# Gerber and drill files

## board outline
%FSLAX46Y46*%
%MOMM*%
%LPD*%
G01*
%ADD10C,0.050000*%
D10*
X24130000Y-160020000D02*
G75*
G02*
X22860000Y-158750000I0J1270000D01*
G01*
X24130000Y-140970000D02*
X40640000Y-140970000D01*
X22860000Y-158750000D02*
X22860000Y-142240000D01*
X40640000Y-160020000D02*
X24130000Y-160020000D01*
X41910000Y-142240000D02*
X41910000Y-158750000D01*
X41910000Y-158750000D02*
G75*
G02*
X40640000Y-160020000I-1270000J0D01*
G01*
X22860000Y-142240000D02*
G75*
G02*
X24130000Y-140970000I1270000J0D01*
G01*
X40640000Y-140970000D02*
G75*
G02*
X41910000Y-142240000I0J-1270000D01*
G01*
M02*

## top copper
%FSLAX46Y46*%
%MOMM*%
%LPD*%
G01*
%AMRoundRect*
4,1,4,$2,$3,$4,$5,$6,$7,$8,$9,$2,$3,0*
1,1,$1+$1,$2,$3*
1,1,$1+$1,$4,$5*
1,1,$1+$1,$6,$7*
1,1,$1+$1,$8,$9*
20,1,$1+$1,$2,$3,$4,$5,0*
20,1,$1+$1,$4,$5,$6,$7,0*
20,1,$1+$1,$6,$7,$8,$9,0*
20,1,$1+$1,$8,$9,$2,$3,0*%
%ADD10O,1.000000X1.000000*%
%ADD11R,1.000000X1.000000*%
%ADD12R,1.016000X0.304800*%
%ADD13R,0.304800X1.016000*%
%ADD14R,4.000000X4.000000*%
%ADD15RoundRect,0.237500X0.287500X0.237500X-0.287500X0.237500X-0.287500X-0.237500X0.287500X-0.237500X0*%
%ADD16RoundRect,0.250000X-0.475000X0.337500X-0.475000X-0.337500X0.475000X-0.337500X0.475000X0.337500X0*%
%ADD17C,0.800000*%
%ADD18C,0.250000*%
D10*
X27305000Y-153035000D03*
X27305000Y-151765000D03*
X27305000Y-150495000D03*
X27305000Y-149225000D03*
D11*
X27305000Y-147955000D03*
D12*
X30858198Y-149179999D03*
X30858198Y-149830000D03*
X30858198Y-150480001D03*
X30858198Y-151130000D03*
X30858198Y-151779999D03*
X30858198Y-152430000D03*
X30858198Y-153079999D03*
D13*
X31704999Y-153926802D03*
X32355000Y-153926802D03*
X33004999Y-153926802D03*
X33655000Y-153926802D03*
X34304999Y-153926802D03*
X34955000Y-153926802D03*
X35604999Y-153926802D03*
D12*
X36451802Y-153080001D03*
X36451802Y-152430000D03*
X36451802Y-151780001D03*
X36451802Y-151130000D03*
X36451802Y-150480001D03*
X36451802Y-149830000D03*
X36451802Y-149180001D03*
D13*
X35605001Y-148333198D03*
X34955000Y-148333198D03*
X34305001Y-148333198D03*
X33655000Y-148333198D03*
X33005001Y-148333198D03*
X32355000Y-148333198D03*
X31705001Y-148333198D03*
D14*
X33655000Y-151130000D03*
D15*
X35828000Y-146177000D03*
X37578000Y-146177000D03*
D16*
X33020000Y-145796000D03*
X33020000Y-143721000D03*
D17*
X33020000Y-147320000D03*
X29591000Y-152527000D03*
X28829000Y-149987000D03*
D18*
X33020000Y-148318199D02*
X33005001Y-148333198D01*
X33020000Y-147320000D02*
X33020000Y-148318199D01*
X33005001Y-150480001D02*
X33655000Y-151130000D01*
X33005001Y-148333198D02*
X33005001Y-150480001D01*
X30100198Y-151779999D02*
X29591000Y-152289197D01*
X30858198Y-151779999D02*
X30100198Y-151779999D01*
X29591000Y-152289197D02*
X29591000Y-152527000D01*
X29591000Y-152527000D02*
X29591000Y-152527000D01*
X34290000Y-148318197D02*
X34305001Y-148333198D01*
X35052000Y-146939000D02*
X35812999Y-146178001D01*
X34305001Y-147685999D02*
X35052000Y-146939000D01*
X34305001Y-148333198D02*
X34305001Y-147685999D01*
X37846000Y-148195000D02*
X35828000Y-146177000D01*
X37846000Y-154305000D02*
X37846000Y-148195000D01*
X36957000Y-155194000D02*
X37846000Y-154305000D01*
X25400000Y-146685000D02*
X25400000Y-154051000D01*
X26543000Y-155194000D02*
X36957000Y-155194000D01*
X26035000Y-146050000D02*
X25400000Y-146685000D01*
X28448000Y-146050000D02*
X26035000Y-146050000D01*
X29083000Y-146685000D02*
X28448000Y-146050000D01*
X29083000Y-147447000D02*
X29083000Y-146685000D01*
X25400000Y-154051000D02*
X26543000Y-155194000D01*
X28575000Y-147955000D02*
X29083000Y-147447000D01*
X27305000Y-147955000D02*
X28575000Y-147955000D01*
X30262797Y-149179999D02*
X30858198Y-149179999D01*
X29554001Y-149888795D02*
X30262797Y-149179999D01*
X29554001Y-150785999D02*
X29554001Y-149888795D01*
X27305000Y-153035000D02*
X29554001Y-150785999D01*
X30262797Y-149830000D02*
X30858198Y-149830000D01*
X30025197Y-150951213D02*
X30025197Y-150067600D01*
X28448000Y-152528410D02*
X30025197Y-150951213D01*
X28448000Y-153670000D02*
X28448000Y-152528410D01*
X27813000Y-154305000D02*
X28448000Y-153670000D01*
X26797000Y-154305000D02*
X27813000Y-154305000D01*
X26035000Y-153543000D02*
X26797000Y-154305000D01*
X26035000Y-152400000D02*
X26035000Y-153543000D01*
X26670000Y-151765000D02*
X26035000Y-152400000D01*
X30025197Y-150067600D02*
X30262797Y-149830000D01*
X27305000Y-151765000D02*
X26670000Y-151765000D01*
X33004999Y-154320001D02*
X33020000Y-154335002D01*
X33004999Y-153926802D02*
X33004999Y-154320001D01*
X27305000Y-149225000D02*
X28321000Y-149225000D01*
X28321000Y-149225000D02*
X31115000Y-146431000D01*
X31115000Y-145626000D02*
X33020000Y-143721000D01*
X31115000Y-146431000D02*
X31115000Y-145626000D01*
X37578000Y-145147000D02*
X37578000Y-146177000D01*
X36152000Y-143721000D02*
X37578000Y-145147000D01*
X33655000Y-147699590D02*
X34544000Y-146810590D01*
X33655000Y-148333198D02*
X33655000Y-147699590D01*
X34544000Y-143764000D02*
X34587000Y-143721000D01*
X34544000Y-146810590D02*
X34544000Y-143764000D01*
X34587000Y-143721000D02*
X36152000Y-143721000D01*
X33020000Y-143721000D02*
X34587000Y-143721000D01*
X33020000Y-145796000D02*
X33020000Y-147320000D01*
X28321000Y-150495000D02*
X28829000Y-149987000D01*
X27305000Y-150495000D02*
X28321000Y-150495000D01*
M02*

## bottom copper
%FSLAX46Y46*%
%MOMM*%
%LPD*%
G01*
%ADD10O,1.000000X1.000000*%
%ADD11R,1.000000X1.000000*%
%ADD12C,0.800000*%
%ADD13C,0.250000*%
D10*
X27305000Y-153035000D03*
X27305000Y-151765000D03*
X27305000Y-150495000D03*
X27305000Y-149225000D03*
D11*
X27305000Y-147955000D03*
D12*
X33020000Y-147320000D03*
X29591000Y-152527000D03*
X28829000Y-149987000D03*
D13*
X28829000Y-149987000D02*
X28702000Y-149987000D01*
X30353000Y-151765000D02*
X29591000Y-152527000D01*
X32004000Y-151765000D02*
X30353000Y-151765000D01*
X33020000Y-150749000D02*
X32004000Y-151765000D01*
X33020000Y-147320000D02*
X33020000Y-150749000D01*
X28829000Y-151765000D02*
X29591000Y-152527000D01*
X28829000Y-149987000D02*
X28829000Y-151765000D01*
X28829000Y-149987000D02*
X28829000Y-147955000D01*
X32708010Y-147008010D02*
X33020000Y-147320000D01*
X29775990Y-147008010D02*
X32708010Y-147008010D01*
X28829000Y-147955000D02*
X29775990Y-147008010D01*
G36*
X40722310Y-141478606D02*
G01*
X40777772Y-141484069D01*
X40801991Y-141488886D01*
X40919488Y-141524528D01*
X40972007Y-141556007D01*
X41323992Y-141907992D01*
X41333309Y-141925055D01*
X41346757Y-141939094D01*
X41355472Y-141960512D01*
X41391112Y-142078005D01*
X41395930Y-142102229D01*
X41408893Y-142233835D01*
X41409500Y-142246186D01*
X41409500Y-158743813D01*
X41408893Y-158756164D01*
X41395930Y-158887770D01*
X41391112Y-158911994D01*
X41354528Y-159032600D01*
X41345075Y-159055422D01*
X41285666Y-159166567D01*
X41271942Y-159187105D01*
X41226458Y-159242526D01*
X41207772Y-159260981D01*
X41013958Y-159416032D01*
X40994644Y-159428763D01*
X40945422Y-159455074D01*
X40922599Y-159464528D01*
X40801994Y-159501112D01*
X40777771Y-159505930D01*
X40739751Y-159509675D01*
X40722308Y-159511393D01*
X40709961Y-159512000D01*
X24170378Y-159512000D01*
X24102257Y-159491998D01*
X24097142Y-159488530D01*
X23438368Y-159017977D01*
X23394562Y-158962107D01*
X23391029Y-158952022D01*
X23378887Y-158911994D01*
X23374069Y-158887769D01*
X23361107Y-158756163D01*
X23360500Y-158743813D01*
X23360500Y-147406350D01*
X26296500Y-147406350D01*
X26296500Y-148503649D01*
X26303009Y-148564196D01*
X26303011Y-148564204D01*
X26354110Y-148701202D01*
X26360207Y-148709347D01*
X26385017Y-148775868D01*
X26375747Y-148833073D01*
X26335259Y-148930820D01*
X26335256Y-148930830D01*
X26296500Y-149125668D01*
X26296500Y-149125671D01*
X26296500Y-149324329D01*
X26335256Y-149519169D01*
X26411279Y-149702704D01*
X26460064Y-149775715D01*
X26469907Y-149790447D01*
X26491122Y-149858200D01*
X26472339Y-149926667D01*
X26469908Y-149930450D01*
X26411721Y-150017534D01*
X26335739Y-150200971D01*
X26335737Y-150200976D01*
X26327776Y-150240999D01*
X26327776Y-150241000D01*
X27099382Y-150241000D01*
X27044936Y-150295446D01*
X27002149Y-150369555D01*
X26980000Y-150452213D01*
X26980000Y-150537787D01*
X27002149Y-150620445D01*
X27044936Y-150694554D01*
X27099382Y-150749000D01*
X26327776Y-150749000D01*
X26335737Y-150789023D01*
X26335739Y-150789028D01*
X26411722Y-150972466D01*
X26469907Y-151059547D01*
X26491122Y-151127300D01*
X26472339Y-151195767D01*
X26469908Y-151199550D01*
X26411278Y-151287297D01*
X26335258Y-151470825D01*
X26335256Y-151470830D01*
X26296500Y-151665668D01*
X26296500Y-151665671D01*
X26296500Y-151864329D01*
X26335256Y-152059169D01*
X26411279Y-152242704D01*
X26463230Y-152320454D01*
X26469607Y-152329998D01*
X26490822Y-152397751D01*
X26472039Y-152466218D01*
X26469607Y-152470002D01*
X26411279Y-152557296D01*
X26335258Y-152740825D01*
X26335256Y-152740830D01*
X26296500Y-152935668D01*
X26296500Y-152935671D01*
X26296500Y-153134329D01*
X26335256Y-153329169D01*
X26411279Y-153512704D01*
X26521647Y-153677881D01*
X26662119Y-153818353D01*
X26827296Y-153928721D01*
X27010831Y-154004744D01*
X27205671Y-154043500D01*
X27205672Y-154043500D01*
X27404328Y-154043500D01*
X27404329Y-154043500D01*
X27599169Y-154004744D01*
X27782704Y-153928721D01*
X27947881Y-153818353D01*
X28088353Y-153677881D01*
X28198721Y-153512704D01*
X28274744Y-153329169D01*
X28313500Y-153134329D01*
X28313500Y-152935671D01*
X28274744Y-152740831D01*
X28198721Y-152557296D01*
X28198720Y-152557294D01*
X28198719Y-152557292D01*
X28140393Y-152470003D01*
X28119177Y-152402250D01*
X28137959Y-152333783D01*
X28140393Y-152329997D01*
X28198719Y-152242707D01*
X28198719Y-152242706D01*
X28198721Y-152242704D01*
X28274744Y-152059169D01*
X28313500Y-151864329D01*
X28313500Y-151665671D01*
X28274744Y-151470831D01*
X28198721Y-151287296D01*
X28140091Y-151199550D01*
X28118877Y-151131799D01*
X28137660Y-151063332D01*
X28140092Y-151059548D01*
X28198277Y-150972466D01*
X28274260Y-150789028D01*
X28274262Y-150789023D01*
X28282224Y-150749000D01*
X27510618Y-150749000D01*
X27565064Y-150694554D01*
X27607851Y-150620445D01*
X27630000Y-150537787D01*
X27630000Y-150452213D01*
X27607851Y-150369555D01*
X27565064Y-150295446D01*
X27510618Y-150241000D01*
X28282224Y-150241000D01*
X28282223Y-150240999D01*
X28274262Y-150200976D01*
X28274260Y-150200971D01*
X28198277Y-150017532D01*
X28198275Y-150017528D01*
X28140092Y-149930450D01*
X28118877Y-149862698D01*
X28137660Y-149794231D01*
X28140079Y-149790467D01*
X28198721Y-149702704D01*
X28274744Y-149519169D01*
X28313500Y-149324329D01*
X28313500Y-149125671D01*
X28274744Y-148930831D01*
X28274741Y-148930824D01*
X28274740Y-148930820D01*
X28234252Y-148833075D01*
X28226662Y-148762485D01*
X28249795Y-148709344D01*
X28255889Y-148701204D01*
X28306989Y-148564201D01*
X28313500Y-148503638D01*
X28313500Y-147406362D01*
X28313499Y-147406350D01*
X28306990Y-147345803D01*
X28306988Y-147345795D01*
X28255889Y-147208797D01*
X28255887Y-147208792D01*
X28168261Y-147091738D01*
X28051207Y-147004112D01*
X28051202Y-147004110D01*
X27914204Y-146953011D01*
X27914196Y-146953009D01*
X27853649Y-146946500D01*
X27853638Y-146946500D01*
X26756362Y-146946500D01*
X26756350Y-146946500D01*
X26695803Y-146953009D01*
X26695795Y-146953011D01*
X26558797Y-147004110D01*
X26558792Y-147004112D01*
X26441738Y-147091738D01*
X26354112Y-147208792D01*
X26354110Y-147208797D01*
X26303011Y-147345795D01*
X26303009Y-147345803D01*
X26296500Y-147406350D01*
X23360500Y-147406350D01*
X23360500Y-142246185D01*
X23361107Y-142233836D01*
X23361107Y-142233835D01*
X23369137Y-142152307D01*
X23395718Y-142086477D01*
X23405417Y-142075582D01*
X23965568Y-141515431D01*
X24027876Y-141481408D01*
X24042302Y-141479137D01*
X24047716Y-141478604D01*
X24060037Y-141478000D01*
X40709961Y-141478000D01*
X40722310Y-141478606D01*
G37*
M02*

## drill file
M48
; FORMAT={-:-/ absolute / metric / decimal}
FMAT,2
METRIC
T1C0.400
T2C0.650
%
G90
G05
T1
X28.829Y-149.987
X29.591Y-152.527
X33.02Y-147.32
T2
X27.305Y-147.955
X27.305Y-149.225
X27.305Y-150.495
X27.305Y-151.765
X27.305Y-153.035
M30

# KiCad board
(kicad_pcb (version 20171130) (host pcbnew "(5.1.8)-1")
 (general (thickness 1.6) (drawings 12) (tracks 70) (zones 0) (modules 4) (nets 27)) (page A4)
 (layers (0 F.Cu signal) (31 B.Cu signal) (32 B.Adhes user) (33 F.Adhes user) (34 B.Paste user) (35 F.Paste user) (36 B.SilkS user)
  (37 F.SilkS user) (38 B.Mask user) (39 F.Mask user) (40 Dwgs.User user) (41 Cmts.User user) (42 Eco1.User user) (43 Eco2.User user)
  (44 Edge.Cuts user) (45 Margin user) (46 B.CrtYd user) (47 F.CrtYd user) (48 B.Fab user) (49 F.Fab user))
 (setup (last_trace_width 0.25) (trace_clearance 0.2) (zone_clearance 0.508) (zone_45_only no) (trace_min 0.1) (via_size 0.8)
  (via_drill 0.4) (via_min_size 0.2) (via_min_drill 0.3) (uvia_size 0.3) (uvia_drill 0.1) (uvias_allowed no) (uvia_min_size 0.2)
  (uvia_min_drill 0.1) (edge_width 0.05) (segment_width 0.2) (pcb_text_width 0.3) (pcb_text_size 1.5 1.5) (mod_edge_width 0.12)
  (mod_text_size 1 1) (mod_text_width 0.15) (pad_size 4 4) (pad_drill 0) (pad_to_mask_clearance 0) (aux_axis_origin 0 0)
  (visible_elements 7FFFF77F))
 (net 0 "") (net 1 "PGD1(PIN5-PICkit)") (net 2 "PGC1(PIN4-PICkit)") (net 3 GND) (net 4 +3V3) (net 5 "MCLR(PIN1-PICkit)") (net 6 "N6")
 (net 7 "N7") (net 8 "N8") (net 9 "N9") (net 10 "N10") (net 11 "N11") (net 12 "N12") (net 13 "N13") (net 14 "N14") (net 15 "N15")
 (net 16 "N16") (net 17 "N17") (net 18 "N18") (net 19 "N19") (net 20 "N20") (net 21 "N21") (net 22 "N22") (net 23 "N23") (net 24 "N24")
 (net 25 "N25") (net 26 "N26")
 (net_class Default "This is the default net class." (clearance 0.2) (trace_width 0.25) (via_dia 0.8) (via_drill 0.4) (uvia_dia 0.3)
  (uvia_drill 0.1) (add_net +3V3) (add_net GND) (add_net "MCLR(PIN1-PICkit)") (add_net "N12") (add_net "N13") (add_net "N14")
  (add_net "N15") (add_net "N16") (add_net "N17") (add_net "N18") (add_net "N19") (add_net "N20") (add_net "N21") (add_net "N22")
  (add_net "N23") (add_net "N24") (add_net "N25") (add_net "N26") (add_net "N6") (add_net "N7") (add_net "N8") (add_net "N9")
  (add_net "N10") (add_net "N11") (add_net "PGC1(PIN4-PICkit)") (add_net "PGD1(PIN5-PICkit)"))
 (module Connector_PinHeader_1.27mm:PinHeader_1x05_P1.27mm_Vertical (layer F.Cu) (at 27.305 147.955)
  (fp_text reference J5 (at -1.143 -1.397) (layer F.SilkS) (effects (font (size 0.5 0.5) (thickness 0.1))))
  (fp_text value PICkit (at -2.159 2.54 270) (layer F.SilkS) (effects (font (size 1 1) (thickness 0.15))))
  (pad 5 thru_hole oval (at 0 5.08) (size 1 1) (drill 0.65) (layers *.Cu *.Mask) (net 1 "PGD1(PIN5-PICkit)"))
  (pad 4 thru_hole oval (at 0 3.81) (size 1 1) (drill 0.65) (layers *.Cu *.Mask) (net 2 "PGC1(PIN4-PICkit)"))
  (pad 3 thru_hole oval (at 0 2.54) (size 1 1) (drill 0.65) (layers *.Cu *.Mask) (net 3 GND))
  (pad 2 thru_hole oval (at 0 1.27) (size 1 1) (drill 0.65) (layers *.Cu *.Mask) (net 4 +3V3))
  (pad 1 thru_hole rect (at 0 0) (size 1 1) (drill 0.65) (layers *.Cu *.Mask) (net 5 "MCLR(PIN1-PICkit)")))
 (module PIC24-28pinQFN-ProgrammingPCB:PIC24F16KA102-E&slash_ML (layer F.Cu) (at 33.655 151.13)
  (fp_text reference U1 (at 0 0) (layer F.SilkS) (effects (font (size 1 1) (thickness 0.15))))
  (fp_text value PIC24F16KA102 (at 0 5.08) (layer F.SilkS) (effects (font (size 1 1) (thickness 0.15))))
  (pad 1 smd rect (at -2.796802 -1.950001 90) (size 0.3048 1.016) (layers F.Cu F.Paste F.Mask) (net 1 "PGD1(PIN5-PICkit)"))
  (pad 2 smd rect (at -2.796802 -1.3 90) (size 0.3048 1.016) (layers F.Cu F.Paste F.Mask) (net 2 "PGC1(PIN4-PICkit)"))
  (pad 3 smd rect (at -2.796802 -0.649999 90) (size 0.3048 1.016) (layers F.Cu F.Paste F.Mask) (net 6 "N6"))
  (pad 4 smd rect (at -2.796802 0 90) (size 0.3048 1.016) (layers F.Cu F.Paste F.Mask) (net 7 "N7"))
  (pad 5 smd rect (at -2.796802 0.649999 90) (size 0.3048 1.016) (layers F.Cu F.Paste F.Mask) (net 3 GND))
  (pad 6 smd rect (at -2.796802 1.3 90) (size 0.3048 1.016) (layers F.Cu F.Paste F.Mask) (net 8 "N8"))
  (pad 7 smd rect (at -2.796802 1.949999 90) (size 0.3048 1.016) (layers F.Cu F.Paste F.Mask) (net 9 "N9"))
  (pad 8 smd rect (at -1.950001 2.796802) (size 0.3048 1.016) (layers F.Cu F.Paste F.Mask) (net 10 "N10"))
  (pad 9 smd rect (at -1.3 2.796802) (size 0.3048 1.016) (layers F.Cu F.Paste F.Mask) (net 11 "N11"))
  (pad 10 smd rect (at -0.650001 2.796802) (size 0.3048 1.016) (layers F.Cu F.Paste F.Mask) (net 4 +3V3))
  (pad 11 smd rect (at 0 2.796802) (size 0.3048 1.016) (layers F.Cu F.Paste F.Mask) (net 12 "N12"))
  (pad 12 smd rect (at 0.649999 2.796802) (size 0.3048 1.016) (layers F.Cu F.Paste F.Mask) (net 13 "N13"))
  (pad 13 smd rect (at 1.3 2.796802) (size 0.3048 1.016) (layers F.Cu F.Paste F.Mask) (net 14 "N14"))
  (pad 14 smd rect (at 1.949999 2.796802) (size 0.3048 1.016) (layers F.Cu F.Paste F.Mask) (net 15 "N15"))
  (pad 15 smd rect (at 2.796802 1.950001 90) (size 0.3048 1.016) (layers F.Cu F.Paste F.Mask) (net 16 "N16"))
  (pad 16 smd rect (at 2.796802 1.3 90) (size 0.3048 1.016) (layers F.Cu F.Paste F.Mask) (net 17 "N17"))
  (pad 17 smd rect (at 2.796802 0.650001 90) (size 0.3048 1.016) (layers F.Cu F.Paste F.Mask) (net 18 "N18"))
  (pad 18 smd rect (at 2.796802 0 90) (size 0.3048 1.016) (layers F.Cu F.Paste F.Mask) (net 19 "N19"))
  (pad 19 smd rect (at 2.796802 -0.649999 90) (size 0.3048 1.016) (layers F.Cu F.Paste F.Mask) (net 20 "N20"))
  (pad 20 smd rect (at 2.796802 -1.3 90) (size 0.3048 1.016) (layers F.Cu F.Paste F.Mask) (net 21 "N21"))
  (pad 21 smd rect (at 2.796802 -1.949999 90) (size 0.3048 1.016) (layers F.Cu F.Paste F.Mask) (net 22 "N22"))
  (pad 22 smd rect (at 1.950001 -2.796802) (size 0.3048 1.016) (layers F.Cu F.Paste F.Mask) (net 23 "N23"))
  (pad 23 smd rect (at 1.3 -2.796802) (size 0.3048 1.016) (layers F.Cu F.Paste F.Mask) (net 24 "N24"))
  (pad 24 smd rect (at 0.650001 -2.796802) (size 0.3048 1.016) (layers F.Cu F.Paste F.Mask) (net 5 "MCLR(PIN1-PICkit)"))
  (pad 25 smd rect (at 0 -2.796802) (size 0.3048 1.016) (layers F.Cu F.Paste F.Mask) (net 4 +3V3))
  (pad 26 smd rect (at -0.649999 -2.796802) (size 0.3048 1.016) (layers F.Cu F.Paste F.Mask) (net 3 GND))
  (pad 27 smd rect (at -1.3 -2.796802) (size 0.3048 1.016) (layers F.Cu F.Paste F.Mask) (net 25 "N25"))
  (pad 28 smd rect (at -1.949999 -2.796802) (size 0.3048 1.016) (layers F.Cu F.Paste F.Mask) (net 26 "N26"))
  (pad EP smd rect (at 0 0) (size 4 4) (layers F.Cu F.Paste F.Mask) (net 3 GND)))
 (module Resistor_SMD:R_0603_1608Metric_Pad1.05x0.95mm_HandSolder (layer F.Cu) (at 36.703 146.177 180)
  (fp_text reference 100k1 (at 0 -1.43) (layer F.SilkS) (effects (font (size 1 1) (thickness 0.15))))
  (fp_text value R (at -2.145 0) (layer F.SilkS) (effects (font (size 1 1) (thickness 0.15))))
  (pad 2 smd roundrect (at 0.875 0 180) (size 1.05 0.95) (layers F.Cu F.Paste F.Mask) (roundrect_rratio 0.25) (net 5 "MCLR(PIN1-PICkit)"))
  (pad 1 smd roundrect (at -0.875 0 180) (size 1.05 0.95) (layers F.Cu F.Paste F.Mask) (roundrect_rratio 0.25) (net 4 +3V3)))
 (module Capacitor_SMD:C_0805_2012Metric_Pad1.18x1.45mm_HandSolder (layer F.Cu) (at 33.02 144.7585 270)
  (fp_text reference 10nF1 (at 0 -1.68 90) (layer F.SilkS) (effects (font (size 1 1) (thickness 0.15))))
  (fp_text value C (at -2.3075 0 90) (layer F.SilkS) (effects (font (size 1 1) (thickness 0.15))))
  (pad 2 smd roundrect (at 1.0375 0 270) (size 1.175 1.45) (layers F.Cu F.Paste F.Mask) (roundrect_rratio 0.212766) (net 3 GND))
  (pad 1 smd roundrect (at -1.0375 0 270) (size 1.175 1.45) (layers F.Cu F.Paste F.Mask) (roundrect_rratio 0.212766) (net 4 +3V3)))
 (gr_arc (start 24.13 158.75) (end 22.86 158.75) (angle -90) (layer Edge.Cuts) (width 0.05))
 (gr_line (start 24.13 140.97) (end 40.64 140.97) (layer Edge.Cuts) (width 0.05))
 (gr_line (start 22.86 158.75) (end 22.86 142.24) (layer Edge.Cuts) (width 0.05))
 (gr_line (start 40.64 160.02) (end 24.13 160.02) (layer Edge.Cuts) (width 0.05))
 (gr_line (start 41.91 142.24) (end 41.91 158.75) (layer Edge.Cuts) (width 0.05))
 (gr_arc (start 40.64 158.75) (end 40.64 160.02) (angle -90) (layer Edge.Cuts) (width 0.05))
 (gr_arc (start 24.13 142.24) (end 24.13 140.97) (angle -90) (layer Edge.Cuts) (width 0.05))
 (gr_arc (start 40.64 142.24) (end 41.91 142.24) (angle -90) (layer Edge.Cuts) (width 0.05))
 (via (at 33.02 147.32) (size 0.8) (drill 0.4) (layers F.Cu B.Cu) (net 3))
 (segment (start 33.02 148.318199) (end 33.005001 148.333198) (width 0.25) (layer F.Cu) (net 3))
 (segment (start 33.02 147.32) (end 33.02 148.318199) (width 0.25) (layer F.Cu) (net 3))
 (segment (start 33.005001 150.480001) (end 33.655 151.13) (width 0.25) (layer F.Cu) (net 3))
 (segment (start 33.005001 148.333198) (end 33.005001 150.480001) (width 0.25) (layer F.Cu) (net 3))
 (segment (start 30.100198 151.779999) (end 29.591 152.289197) (width 0.25) (layer F.Cu) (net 3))
 (segment (start 30.858198 151.779999) (end 30.100198 151.779999) (width 0.25) (layer F.Cu) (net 3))
 (segment (start 29.591 152.289197) (end 29.591 152.527) (width 0.25) (layer F.Cu) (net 3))
 (segment (start 29.591 152.527) (end 29.591 152.527) (width 0.25) (layer F.Cu) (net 3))
 (via (at 29.591 152.527) (size 0.8) (drill 0.4) (layers F.Cu B.Cu) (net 3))
 (segment (start 34.29 148.318197) (end 34.305001 148.333198) (width 0.25) (layer F.Cu) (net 5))
 (segment (start 35.052 146.939) (end 35.812999 146.178001) (width 0.25) (layer F.Cu) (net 5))
 (segment (start 34.305001 147.685999) (end 35.052 146.939) (width 0.25) (layer F.Cu) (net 5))
 (segment (start 34.305001 148.333198) (end 34.305001 147.685999) (width 0.25) (layer F.Cu) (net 5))
 (segment (start 37.846 148.195) (end 35.828 146.177) (width 0.25) (layer F.Cu) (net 5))
 (segment (start 37.846 154.305) (end 37.846 148.195) (width 0.25) (layer F.Cu) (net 5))
 (segment (start 36.957 155.194) (end 37.846 154.305) (width 0.25) (layer F.Cu) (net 5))
 (segment (start 25.4 146.685) (end 25.4 154.051) (width 0.25) (layer F.Cu) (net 5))
 (segment (start 26.543 155.194) (end 36.957 155.194) (width 0.25) (layer F.Cu) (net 5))
 (segment (start 26.035 146.05) (end 25.4 146.685) (width 0.25) (layer F.Cu) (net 5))
 (segment (start 28.448 146.05) (end 26.035 146.05) (width 0.25) (layer F.Cu) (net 5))
 (segment (start 29.083 146.685) (end 28.448 146.05) (width 0.25) (layer F.Cu) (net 5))
 (segment (start 29.083 147.447) (end 29.083 146.685) (width 0.25) (layer F.Cu) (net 5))
 (segment (start 25.4 154.051) (end 26.543 155.194) (width 0.25) (layer F.Cu) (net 5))
 (segment (start 28.575 147.955) (end 29.083 147.447) (width 0.25) (layer F.Cu) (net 5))
 (segment (start 27.305 147.955) (end 28.575 147.955) (width 0.25) (layer F.Cu) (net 5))
 (segment (start 30.262797 149.179999) (end 30.858198 149.179999) (width 0.25) (layer F.Cu) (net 1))
 (segment (start 29.554001 149.888795) (end 30.262797 149.179999) (width 0.25) (layer F.Cu) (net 1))
 (segment (start 29.554001 150.785999) (end 29.554001 149.888795) (width 0.25) (layer F.Cu) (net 1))
 (segment (start 27.305 153.035) (end 29.554001 150.785999) (width 0.25) (layer F.Cu) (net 1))
 (segment (start 30.262797 149.83) (end 30.858198 149.83) (width 0.25) (layer F.Cu) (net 2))
 (segment (start 30.025197 150.951213) (end 30.025197 150.0676) (width 0.25) (layer F.Cu) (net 2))
 (segment (start 28.448 152.52841) (end 30.025197 150.951213) (width 0.25) (layer F.Cu) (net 2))
 (segment (start 28.448 153.67) (end 28.448 152.52841) (width 0.25) (layer F.Cu) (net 2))
 (segment (start 27.813 154.305) (end 28.448 153.67) (width 0.25) (layer F.Cu) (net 2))
 (segment (start 26.797 154.305) (end 27.813 154.305) (width 0.25) (layer F.Cu) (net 2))
 (segment (start 26.035 153.543) (end 26.797 154.305) (width 0.25) (layer F.Cu) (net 2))
 (segment (start 26.035 152.4) (end 26.035 153.543) (width 0.25) (layer F.Cu) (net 2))
 (segment (start 26.67 151.765) (end 26.035 152.4) (width 0.25) (layer F.Cu) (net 2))
 (segment (start 30.025197 150.0676) (end 30.262797 149.83) (width 0.25) (layer F.Cu) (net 2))
 (segment (start 27.305 151.765) (end 26.67 151.765) (width 0.25) (layer F.Cu) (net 2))
 (segment (start 33.004999 154.320001) (end 33.02 154.335002) (width 0.25) (layer F.Cu) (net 4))
 (segment (start 33.004999 153.926802) (end 33.004999 154.320001) (width 0.25) (layer F.Cu) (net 4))
 (segment (start 27.305 149.225) (end 28.321 149.225) (width 0.25) (layer F.Cu) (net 4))
 (segment (start 28.321 149.225) (end 31.115 146.431) (width 0.25) (layer F.Cu) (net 4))
 (segment (start 31.115 145.626) (end 33.02 143.721) (width 0.25) (layer F.Cu) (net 4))
 (segment (start 31.115 146.431) (end 31.115 145.626) (width 0.25) (layer F.Cu) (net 4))
 (segment (start 37.578 145.147) (end 37.578 146.177) (width 0.25) (layer F.Cu) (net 4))
 (segment (start 36.152 143.721) (end 37.578 145.147) (width 0.25) (layer F.Cu) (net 4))
 (segment (start 33.655 147.69959) (end 34.544 146.81059) (width 0.25) (layer F.Cu) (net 4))
 (segment (start 33.655 148.333198) (end 33.655 147.69959) (width 0.25) (layer F.Cu) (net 4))
 (segment (start 34.544 143.764) (end 34.587 143.721) (width 0.25) (layer F.Cu) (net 4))
 (segment (start 34.544 146.81059) (end 34.544 143.764) (width 0.25) (layer F.Cu) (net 4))
 (segment (start 34.587 143.721) (end 36.152 143.721) (width 0.25) (layer F.Cu) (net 4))
 (segment (start 33.02 143.721) (end 34.587 143.721) (width 0.25) (layer F.Cu) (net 4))
 (segment (start 33.02 145.796) (end 33.02 147.32) (width 0.25) (layer F.Cu) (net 3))
 (segment (start 28.829 149.987) (end 28.702 149.987) (width 0.25) (layer B.Cu) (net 3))
 (via (at 28.829 149.987) (size 0.8) (drill 0.4) (layers F.Cu B.Cu) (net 3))
 (segment (start 28.321 150.495) (end 28.829 149.987) (width 0.25) (layer F.Cu) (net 3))
 (segment (start 27.305 150.495) (end 28.321 150.495) (width 0.25) (layer F.Cu) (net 3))
 (segment (start 30.353 151.765) (end 29.591 152.527) (width 0.25) (layer B.Cu) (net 3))
 (segment (start 32.004 151.765) (end 30.353 151.765) (width 0.25) (layer B.Cu) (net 3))
 (segment (start 33.02 150.749) (end 32.004 151.765) (width 0.25) (layer B.Cu) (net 3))
 (segment (start 33.02 147.32) (end 33.02 150.749) (width 0.25) (layer B.Cu) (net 3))
 (segment (start 28.829 151.765) (end 29.591 152.527) (width 0.25) (layer B.Cu) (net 3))
 (segment (start 28.829 149.987) (end 28.829 151.765) (width 0.25) (layer B.Cu) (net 3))
 (segment (start 28.829 149.987) (end 28.829 147.955) (width 0.25) (layer B.Cu) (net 3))
 (segment (start 32.70801 147.00801) (end 33.02 147.32) (width 0.25) (layer B.Cu) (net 3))
 (segment (start 29.77599 147.00801) (end 32.70801 147.00801) (width 0.25) (layer B.Cu) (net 3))
 (segment (start 28.829 147.955) (end 29.77599 147.00801) (width 0.25) (layer B.Cu) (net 3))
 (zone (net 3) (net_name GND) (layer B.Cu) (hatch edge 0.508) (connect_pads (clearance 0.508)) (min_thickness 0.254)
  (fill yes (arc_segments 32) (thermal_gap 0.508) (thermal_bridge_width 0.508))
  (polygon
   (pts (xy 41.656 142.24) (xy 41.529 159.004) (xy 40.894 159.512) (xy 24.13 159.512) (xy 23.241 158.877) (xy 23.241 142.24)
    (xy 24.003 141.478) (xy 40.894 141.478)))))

